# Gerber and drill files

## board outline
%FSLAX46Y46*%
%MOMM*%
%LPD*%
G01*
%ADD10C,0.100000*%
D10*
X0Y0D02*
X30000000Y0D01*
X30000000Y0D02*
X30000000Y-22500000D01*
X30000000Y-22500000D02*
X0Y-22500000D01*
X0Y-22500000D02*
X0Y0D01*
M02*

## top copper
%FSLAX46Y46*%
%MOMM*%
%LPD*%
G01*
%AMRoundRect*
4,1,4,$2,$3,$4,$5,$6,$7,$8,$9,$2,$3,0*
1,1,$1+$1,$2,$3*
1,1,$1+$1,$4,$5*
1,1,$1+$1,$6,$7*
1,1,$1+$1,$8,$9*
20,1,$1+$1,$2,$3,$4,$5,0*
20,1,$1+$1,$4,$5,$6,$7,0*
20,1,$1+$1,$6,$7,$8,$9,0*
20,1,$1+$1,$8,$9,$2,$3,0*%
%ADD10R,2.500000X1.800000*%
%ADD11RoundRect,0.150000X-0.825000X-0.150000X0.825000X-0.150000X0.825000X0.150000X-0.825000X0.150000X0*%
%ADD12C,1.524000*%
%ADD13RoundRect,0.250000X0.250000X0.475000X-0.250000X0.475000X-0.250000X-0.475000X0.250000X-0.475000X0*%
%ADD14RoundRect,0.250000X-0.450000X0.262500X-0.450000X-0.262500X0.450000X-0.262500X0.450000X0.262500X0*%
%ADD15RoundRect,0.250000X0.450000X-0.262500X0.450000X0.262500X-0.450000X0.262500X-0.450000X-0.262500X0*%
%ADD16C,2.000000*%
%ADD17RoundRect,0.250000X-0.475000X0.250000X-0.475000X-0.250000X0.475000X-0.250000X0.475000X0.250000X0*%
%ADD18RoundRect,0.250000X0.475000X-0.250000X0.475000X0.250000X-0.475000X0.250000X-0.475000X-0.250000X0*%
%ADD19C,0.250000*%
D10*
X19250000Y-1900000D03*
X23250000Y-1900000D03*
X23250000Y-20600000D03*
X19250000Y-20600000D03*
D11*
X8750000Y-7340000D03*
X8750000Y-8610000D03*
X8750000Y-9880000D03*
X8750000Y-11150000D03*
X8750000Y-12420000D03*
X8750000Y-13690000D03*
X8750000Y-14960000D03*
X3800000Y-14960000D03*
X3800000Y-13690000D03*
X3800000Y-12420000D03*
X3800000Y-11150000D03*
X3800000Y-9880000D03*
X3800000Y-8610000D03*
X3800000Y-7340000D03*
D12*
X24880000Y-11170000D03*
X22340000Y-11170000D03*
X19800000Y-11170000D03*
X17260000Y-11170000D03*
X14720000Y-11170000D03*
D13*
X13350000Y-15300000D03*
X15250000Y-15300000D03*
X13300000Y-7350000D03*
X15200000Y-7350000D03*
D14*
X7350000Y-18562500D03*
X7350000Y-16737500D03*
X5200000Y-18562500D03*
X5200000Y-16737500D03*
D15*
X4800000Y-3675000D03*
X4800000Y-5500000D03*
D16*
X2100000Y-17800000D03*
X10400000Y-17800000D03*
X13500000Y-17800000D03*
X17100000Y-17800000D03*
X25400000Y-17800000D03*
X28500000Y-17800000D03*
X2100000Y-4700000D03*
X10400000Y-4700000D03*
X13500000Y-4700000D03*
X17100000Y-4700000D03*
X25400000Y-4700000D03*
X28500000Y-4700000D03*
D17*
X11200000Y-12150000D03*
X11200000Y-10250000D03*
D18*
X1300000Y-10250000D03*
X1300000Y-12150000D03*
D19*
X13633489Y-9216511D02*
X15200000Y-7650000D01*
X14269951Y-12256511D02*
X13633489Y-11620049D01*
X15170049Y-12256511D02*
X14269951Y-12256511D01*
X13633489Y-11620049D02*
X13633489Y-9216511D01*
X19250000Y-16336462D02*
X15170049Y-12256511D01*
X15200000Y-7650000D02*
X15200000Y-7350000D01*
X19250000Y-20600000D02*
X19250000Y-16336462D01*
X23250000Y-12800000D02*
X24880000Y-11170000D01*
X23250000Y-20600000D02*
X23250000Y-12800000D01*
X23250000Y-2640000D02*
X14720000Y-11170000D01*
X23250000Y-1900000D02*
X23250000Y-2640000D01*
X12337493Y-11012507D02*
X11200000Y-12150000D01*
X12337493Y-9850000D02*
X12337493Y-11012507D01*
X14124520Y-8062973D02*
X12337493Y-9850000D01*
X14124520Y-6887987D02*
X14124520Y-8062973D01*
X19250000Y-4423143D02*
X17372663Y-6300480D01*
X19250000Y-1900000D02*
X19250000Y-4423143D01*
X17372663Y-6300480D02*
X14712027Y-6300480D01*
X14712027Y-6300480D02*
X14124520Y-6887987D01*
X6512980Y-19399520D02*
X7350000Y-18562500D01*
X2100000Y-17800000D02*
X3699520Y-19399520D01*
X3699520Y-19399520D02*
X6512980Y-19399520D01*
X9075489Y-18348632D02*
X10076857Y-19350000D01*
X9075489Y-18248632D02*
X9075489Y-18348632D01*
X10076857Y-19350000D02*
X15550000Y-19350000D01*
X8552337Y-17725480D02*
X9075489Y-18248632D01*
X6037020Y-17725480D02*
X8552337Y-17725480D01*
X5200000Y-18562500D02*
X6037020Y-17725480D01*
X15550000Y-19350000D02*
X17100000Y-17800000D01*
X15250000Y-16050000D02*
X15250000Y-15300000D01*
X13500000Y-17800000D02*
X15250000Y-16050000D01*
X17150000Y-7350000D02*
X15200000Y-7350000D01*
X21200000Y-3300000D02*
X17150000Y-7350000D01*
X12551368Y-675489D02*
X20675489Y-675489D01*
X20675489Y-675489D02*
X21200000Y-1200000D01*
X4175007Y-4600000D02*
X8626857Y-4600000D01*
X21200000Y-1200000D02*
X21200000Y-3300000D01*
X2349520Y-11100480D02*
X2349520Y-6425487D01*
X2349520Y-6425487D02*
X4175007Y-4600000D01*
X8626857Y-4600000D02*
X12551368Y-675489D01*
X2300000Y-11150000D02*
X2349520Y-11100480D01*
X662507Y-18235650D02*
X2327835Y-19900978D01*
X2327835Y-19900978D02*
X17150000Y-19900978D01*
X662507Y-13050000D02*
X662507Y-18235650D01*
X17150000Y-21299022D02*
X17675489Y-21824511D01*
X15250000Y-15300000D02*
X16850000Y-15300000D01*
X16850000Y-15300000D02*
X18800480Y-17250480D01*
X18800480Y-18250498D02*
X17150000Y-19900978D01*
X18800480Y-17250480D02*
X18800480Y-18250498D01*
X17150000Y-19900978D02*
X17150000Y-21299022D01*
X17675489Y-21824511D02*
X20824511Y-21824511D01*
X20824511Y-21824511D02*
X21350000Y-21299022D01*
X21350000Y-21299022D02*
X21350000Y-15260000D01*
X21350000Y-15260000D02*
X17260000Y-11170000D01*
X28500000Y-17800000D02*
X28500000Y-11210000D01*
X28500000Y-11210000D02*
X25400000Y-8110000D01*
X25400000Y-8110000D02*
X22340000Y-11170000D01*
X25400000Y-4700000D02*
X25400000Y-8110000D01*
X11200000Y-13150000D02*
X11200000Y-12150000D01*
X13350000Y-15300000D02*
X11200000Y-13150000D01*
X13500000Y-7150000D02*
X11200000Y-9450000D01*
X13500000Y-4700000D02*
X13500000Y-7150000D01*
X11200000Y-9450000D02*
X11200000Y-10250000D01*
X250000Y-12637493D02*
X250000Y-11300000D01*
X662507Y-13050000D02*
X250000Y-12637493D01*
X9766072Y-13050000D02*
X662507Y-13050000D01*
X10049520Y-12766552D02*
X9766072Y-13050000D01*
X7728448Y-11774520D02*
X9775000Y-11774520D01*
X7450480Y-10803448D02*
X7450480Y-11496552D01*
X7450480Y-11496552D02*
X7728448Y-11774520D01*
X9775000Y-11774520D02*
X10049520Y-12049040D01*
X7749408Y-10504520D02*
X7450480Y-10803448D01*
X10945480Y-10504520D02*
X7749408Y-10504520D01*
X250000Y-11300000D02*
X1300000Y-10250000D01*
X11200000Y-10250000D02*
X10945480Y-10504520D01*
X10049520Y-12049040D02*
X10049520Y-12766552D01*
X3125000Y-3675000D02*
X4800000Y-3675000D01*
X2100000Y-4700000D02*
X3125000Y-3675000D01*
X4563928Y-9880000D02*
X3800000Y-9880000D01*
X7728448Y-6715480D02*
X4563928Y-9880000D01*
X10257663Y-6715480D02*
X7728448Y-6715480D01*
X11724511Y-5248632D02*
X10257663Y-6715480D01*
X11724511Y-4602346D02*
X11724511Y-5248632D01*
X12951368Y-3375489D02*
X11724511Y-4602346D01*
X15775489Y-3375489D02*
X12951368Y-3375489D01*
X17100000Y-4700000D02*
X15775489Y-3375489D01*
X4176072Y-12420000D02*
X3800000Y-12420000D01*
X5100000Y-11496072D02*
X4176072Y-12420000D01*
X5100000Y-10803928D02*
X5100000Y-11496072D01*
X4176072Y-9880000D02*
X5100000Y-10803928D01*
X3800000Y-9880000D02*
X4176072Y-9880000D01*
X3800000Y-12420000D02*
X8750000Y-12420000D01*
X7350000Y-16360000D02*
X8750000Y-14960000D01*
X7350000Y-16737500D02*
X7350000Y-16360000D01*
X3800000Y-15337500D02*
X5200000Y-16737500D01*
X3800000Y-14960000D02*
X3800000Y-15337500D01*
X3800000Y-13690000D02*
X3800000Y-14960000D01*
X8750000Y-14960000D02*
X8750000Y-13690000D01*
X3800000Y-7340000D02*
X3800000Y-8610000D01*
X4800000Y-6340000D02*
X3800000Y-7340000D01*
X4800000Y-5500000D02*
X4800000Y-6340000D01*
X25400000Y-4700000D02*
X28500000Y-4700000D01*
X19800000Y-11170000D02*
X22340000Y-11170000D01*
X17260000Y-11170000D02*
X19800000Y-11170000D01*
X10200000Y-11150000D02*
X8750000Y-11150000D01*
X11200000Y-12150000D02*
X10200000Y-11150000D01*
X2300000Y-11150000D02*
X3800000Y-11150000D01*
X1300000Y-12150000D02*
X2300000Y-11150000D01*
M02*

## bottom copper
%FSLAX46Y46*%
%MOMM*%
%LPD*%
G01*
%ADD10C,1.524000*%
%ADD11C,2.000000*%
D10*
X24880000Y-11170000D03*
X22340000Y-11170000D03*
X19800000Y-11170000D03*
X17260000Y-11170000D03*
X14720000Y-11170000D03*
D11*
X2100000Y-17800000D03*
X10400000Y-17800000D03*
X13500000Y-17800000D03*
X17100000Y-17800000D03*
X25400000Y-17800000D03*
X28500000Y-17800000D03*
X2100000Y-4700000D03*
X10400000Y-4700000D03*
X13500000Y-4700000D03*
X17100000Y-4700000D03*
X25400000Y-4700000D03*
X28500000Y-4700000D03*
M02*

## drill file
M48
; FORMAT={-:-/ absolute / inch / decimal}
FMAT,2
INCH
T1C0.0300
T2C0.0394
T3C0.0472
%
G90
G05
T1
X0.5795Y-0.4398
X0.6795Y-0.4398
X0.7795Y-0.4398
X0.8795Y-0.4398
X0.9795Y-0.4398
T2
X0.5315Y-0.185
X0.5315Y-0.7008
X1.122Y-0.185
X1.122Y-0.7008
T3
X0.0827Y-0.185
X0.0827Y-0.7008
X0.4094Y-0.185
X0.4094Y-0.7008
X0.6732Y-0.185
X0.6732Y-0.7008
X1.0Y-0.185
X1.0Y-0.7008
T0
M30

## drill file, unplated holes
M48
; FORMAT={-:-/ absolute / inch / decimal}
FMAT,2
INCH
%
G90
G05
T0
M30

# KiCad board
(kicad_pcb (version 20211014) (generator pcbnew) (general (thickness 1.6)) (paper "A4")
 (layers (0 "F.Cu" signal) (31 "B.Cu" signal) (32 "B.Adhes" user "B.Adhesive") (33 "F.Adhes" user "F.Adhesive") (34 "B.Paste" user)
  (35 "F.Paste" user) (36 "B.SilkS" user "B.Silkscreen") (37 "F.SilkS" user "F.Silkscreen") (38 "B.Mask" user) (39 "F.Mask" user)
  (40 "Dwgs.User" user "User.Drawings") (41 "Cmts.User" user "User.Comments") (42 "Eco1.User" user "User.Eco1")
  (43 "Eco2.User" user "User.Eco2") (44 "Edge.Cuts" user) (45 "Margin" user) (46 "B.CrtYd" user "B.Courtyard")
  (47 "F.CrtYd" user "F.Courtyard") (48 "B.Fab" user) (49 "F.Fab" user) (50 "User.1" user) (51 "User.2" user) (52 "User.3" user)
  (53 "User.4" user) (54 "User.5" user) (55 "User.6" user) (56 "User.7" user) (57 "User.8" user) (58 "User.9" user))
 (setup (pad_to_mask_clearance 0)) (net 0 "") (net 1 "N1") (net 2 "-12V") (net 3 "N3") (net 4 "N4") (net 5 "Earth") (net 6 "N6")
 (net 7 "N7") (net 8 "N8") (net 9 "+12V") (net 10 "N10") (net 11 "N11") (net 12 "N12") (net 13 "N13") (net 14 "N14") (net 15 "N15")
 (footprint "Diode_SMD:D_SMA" (layer "F.Cu") (at 21.25 1.9 180)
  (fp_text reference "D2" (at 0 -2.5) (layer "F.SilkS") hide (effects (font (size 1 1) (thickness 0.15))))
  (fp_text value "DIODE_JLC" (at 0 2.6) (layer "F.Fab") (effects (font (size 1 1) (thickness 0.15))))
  (pad "1" smd rect (at -2 0 180) (size 2.5 1.8) (layers "F.Cu" "F.Paste" "F.Mask") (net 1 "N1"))
  (pad "2" smd rect (at 2 0 180) (size 2.5 1.8) (layers "F.Cu" "F.Paste" "F.Mask") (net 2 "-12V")))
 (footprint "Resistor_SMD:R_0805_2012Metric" (layer "F.Cu") (at 7.35 17.65 -90)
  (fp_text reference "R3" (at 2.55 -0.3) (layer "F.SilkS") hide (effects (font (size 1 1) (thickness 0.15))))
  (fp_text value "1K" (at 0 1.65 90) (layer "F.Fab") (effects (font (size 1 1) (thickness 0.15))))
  (pad "1" smd roundrect (at -0.9125 0 270) (size 1.025 1.4) (layers "F.Cu" "F.Paste" "F.Mask") (roundrect_rratio 0.243902439) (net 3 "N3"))
  (pad "2" smd roundrect (at 0.9125 0 270) (size 1.025 1.4) (layers "F.Cu" "F.Paste" "F.Mask") (roundrect_rratio 0.243902439) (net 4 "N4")))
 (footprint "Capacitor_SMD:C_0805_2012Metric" (layer "F.Cu") (at 14.3 15.3 180)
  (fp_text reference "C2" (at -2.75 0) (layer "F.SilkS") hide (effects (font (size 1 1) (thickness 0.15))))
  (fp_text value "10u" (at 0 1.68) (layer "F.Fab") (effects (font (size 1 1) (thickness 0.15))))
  (pad "1" smd roundrect (at -0.95 0 180) (size 1 1.45) (layers "F.Cu" "F.Paste" "F.Mask") (roundrect_rratio 0.25) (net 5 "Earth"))
  (pad "2" smd roundrect (at 0.95 0 180) (size 1 1.45) (layers "F.Cu" "F.Paste" "F.Mask") (roundrect_rratio 0.25) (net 2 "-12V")))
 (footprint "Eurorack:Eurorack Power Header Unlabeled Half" (layer "F.Cu") (at 19.8 9.9 180)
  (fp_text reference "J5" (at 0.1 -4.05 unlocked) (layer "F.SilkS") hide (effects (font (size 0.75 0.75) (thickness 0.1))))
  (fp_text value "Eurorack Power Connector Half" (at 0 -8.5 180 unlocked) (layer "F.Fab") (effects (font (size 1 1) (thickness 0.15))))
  (pad "1" thru_hole circle (at 5.08 -1.27 180) (size 1.524 1.524) (drill 0.762) (layers *.Cu *.Mask) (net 1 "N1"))
  (pad "2" thru_hole circle (at 2.54 -1.27 180) (size 1.524 1.524) (drill 0.762) (layers *.Cu *.Mask) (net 5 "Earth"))
  (pad "3" thru_hole circle (at 0 -1.27 180) (size 1.524 1.524) (drill 0.762) (layers *.Cu *.Mask) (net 5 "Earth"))
  (pad "4" thru_hole circle (at -2.54 -1.27 180) (size 1.524 1.524) (drill 0.762) (layers *.Cu *.Mask) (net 5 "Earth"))
  (pad "5" thru_hole circle (at -5.08 -1.27 180) (size 1.524 1.524) (drill 0.762) (layers *.Cu *.Mask) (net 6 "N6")))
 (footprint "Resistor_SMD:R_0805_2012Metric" (layer "F.Cu") (at 5.2 17.65 -90)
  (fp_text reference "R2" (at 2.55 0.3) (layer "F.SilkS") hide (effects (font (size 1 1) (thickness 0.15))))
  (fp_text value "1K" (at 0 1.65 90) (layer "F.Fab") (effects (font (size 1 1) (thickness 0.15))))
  (pad "1" smd roundrect (at -0.9125 0 270) (size 1.025 1.4) (layers "F.Cu" "F.Paste" "F.Mask") (roundrect_rratio 0.243902439) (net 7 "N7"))
  (pad "2" smd roundrect (at 0.9125 0 270) (size 1.025 1.4) (layers "F.Cu" "F.Paste" "F.Mask") (roundrect_rratio 0.243902439) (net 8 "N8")))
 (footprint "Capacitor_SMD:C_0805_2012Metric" (layer "F.Cu") (at 14.25 7.35 180)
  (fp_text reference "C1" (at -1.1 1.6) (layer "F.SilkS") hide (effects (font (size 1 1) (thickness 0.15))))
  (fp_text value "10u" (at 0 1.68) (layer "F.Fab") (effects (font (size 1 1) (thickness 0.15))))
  (pad "1" smd roundrect (at -0.95 0 180) (size 1 1.45) (layers "F.Cu" "F.Paste" "F.Mask") (roundrect_rratio 0.25) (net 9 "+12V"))
  (pad "2" smd roundrect (at 0.95 0 180) (size 1 1.45) (layers "F.Cu" "F.Paste" "F.Mask") (roundrect_rratio 0.25) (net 5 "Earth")))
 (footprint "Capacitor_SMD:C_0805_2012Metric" (layer "F.Cu") (at 11.2 11.2 -90)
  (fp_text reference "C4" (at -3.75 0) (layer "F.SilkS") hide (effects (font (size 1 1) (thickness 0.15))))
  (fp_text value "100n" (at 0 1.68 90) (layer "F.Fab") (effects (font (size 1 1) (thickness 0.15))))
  (pad "1" smd roundrect (at -0.95 0 270) (size 1 1.45) (layers "F.Cu" "F.Paste" "F.Mask") (roundrect_rratio 0.25) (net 5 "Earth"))
  (pad "2" smd roundrect (at 0.95 0 270) (size 1 1.45) (layers "F.Cu" "F.Paste" "F.Mask") (roundrect_rratio 0.25) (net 2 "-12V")))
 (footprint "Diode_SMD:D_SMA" (layer "F.Cu") (at 21.25 20.6)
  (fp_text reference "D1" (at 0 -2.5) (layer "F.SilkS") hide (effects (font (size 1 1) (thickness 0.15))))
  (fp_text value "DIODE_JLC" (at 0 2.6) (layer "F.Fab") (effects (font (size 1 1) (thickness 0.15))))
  (pad "1" smd rect (at -2 0) (size 2.5 1.8) (layers "F.Cu" "F.Paste" "F.Mask") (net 9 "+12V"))
  (pad "2" smd rect (at 2 0) (size 2.5 1.8) (layers "F.Cu" "F.Paste" "F.Mask") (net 6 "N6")))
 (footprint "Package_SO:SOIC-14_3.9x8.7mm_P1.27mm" (layer "F.Cu") (at 6.275 11.15)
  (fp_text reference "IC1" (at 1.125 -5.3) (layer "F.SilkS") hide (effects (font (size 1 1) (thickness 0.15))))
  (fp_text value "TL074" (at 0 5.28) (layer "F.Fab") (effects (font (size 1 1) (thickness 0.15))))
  (pad "1" smd roundrect (at -2.475 -3.81) (size 1.95 0.6) (layers "F.Cu" "F.Paste" "F.Mask") (roundrect_rratio 0.25) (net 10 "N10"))
  (pad "2" smd roundrect (at -2.475 -2.54) (size 1.95 0.6) (layers "F.Cu" "F.Paste" "F.Mask") (roundrect_rratio 0.25) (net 10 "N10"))
  (pad "3" smd roundrect (at -2.475 -1.27) (size 1.95 0.6) (layers "F.Cu" "F.Paste" "F.Mask") (roundrect_rratio 0.25) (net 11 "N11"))
  (pad "4" smd roundrect (at -2.475 0) (size 1.95 0.6) (layers "F.Cu" "F.Paste" "F.Mask") (roundrect_rratio 0.25) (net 9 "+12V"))
  (pad "5" smd roundrect (at -2.475 1.27) (size 1.95 0.6) (layers "F.Cu" "F.Paste" "F.Mask") (roundrect_rratio 0.25) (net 11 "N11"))
  (pad "6" smd roundrect (at -2.475 2.54) (size 1.95 0.6) (layers "F.Cu" "F.Paste" "F.Mask") (roundrect_rratio 0.25) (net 7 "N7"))
  (pad "7" smd roundrect (at -2.475 3.81) (size 1.95 0.6) (layers "F.Cu" "F.Paste" "F.Mask") (roundrect_rratio 0.25) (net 7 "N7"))
  (pad "8" smd roundrect (at 2.475 3.81) (size 1.95 0.6) (layers "F.Cu" "F.Paste" "F.Mask") (roundrect_rratio 0.25) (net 3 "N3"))
  (pad "9" smd roundrect (at 2.475 2.54) (size 1.95 0.6) (layers "F.Cu" "F.Paste" "F.Mask") (roundrect_rratio 0.25) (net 3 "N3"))
  (pad "10" smd roundrect (at 2.475 1.27) (size 1.95 0.6) (layers "F.Cu" "F.Paste" "F.Mask") (roundrect_rratio 0.25) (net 11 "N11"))
  (pad "11" smd roundrect (at 2.475 0) (size 1.95 0.6) (layers "F.Cu" "F.Paste" "F.Mask") (roundrect_rratio 0.25) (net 2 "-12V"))
  (pad "12" smd roundrect (at 2.475 -1.27) (size 1.95 0.6) (layers "F.Cu" "F.Paste" "F.Mask") (roundrect_rratio 0.25))
  (pad "13" smd roundrect (at 2.475 -2.54) (size 1.95 0.6) (layers "F.Cu" "F.Paste" "F.Mask") (roundrect_rratio 0.25))
  (pad "14" smd roundrect (at 2.475 -3.81) (size 1.95 0.6) (layers "F.Cu" "F.Paste" "F.Mask") (roundrect_rratio 0.25)))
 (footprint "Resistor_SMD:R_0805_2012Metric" (layer "F.Cu") (at 4.8 4.5875 90)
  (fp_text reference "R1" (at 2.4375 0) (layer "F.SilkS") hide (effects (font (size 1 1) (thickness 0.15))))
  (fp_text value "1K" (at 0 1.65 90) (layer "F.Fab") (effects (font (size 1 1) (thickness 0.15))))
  (pad "1" smd roundrect (at -0.9125 0 90) (size 1.025 1.4) (layers "F.Cu" "F.Paste" "F.Mask") (roundrect_rratio 0.243902439) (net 10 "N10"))
  (pad "2" smd roundrect (at 0.9125 0 90) (size 1.025 1.4) (layers "F.Cu" "F.Paste" "F.Mask") (roundrect_rratio 0.243902439) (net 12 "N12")))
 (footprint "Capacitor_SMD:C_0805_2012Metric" (layer "F.Cu") (at 1.3 11.2 90)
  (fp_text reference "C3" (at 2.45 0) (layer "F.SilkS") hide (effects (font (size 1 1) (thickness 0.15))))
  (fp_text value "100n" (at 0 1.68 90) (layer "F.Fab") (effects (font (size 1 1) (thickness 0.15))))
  (pad "1" smd roundrect (at -0.95 0 90) (size 1 1.45) (layers "F.Cu" "F.Paste" "F.Mask") (roundrect_rratio 0.25) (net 9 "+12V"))
  (pad "2" smd roundrect (at 0.95 0 90) (size 1 1.45) (layers "F.Cu" "F.Paste" "F.Mask") (roundrect_rratio 0.25) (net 5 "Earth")))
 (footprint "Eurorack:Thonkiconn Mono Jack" (layer "B.Cu") (at 22.5 4.7 180)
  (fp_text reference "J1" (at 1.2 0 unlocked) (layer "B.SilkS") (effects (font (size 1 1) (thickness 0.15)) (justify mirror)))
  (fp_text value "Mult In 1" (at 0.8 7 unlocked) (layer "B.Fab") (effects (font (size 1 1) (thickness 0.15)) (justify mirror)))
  (pad "1" thru_hole circle (at -6 0 180) (size 2 2) (drill 1) (layers *.Cu *.Mask) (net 5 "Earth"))
  (pad "2" thru_hole circle (at -2.9 0 180) (size 2 2) (drill 1.2) (layers *.Cu *.Mask) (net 5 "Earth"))
  (pad "3" thru_hole circle (at 5.4 0 180) (size 2 2) (drill 1.2) (layers *.Cu *.Mask) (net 11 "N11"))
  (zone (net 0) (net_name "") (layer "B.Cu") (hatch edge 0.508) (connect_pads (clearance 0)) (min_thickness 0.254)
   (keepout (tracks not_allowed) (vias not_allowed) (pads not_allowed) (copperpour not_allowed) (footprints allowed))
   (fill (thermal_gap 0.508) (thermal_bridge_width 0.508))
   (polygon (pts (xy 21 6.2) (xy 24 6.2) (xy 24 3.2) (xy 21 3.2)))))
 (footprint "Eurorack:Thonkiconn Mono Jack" (layer "B.Cu") (at 7.5 17.8 180)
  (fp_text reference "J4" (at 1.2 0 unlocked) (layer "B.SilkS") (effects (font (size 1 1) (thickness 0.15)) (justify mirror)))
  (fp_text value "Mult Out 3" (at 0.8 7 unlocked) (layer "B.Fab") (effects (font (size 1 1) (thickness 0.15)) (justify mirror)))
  (pad "1" thru_hole circle (at -6 0 180) (size 2 2) (drill 1) (layers *.Cu *.Mask) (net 5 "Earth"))
  (pad "2" thru_hole circle (at -2.9 0 180) (size 2 2) (drill 1.2) (layers *.Cu *.Mask) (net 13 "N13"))
  (pad "3" thru_hole circle (at 5.4 0 180) (size 2 2) (drill 1.2) (layers *.Cu *.Mask) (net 4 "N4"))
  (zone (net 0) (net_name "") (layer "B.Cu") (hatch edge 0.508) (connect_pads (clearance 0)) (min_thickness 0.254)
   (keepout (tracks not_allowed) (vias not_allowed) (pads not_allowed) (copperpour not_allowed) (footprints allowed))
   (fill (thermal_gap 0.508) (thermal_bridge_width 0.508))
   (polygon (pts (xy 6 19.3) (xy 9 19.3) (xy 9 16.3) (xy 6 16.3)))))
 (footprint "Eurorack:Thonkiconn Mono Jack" (layer "B.Cu") (at 22.5 17.8 180)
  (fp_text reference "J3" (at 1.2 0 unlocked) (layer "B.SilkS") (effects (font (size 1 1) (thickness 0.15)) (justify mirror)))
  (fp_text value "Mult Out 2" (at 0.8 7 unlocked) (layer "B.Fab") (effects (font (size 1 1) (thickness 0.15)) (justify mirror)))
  (pad "1" thru_hole circle (at -6 0 180) (size 2 2) (drill 1) (layers *.Cu *.Mask) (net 5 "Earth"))
  (pad "2" thru_hole circle (at -2.9 0 180) (size 2 2) (drill 1.2) (layers *.Cu *.Mask) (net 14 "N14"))
  (pad "3" thru_hole circle (at 5.4 0 180) (size 2 2) (drill 1.2) (layers *.Cu *.Mask) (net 8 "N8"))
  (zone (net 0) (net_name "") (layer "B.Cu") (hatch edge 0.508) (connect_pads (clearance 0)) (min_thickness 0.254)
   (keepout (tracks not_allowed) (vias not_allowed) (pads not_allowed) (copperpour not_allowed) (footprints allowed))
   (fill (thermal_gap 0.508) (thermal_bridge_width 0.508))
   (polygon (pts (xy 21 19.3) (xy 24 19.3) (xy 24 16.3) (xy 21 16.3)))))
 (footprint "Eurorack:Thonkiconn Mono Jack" (layer "B.Cu") (at 7.5 4.7 180)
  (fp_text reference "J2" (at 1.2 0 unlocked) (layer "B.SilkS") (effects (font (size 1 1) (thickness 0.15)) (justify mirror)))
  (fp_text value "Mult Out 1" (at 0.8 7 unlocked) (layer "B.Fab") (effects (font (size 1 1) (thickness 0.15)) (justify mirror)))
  (pad "1" thru_hole circle (at -6 0 180) (size 2 2) (drill 1) (layers *.Cu *.Mask) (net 5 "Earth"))
  (pad "2" thru_hole circle (at -2.9 0 180) (size 2 2) (drill 1.2) (layers *.Cu *.Mask) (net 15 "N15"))
  (pad "3" thru_hole circle (at 5.4 0 180) (size 2 2) (drill 1.2) (layers *.Cu *.Mask) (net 12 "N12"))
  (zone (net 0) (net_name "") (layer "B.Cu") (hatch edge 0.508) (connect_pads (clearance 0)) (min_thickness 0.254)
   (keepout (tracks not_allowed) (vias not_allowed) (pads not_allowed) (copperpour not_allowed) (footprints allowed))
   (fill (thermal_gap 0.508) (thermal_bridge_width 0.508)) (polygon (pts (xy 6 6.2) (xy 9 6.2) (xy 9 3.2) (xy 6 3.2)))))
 (gr_rect (start 0 0) (end 30 22.5) (layer "Edge.Cuts") (width 0.1) (fill none))
 (segment (start 2.34952 6.425487) (end 4.175007 4.6) (width 0.25) (layer "F.Cu") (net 9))
 (segment (start 2.3 11.15) (end 2.34952 11.10048) (width 0.25) (layer "F.Cu") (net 9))
 (segment (start 20.675489 0.675489) (end 21.2 1.2) (width 0.25) (layer "F.Cu") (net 9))
 (segment (start 8.626857 4.6) (end 12.551368 0.675489) (width 0.25) (layer "F.Cu") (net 9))
 (segment (start 15.170049 12.256511) (end 14.269951 12.256511) (width 0.25) (layer "F.Cu") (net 9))
 (segment (start 21.2 3.3) (end 17.15 7.35) (width 0.25) (layer "F.Cu") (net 9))
 (segment (start 21.2 1.2) (end 21.2 3.3) (width 0.25) (layer "F.Cu") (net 9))
 (segment (start 12.551368 0.675489) (end 20.675489 0.675489) (width 0.25) (layer "F.Cu") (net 9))
 (segment (start 19.25 20.6) (end 19.25 16.336462) (width 0.25) (layer "F.Cu") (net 9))
 (segment (start 14.269951 12.256511) (end 13.633489 11.620049) (width 0.25) (layer "F.Cu") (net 9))
 (segment (start 15.2 7.65) (end 15.2 7.35) (width 0.25) (layer "F.Cu") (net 9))
 (segment (start 13.633489 9.216511) (end 15.2 7.65) (width 0.25) (layer "F.Cu") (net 9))
 (segment (start 19.25 16.336462) (end 15.170049 12.256511) (width 0.25) (layer "F.Cu") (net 9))
 (segment (start 1.3 12.15) (end 2.3 11.15) (width 0.25) (layer "F.Cu") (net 9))
 (segment (start 17.15 7.35) (end 15.2 7.35) (width 0.25) (layer "F.Cu") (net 9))
 (segment (start 2.3 11.15) (end 3.8 11.15) (width 0.25) (layer "F.Cu") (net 9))
 (segment (start 13.633489 11.620049) (end 13.633489 9.216511) (width 0.25) (layer "F.Cu") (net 9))
 (segment (start 4.175007 4.6) (end 8.626857 4.6) (width 0.25) (layer "F.Cu") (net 9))
 (segment (start 2.34952 11.10048) (end 2.34952 6.425487) (width 0.25) (layer "F.Cu") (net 9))
 (segment (start 9.775 11.77452) (end 10.04952 12.04904) (width 0.25) (layer "F.Cu") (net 5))
 (segment (start 10.04952 12.04904) (end 10.04952 12.766552) (width 0.25) (layer "F.Cu") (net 5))
 (segment (start 25.4 4.7) (end 28.5 4.7) (width 0.25) (layer "F.Cu") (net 5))
 (segment (start 0.25 11.3) (end 1.3 10.25) (width 0.25) (layer "F.Cu") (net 5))
 (segment (start 21.35 21.299022) (end 21.35 15.26) (width 0.25) (layer "F.Cu") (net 5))
 (segment (start 7.45048 11.496552) (end 7.728448 11.77452) (width 0.25) (layer "F.Cu") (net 5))
 (segment (start 2.327835 19.900978) (end 17.15 19.900978) (width 0.25) (layer "F.Cu") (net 5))
 (segment (start 18.80048 17.25048) (end 18.80048 18.250498) (width 0.25) (layer "F.Cu") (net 5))
 (segment (start 11.2 10.25) (end 10.94548 10.50452) (width 0.25) (layer "F.Cu") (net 5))
 (segment (start 7.45048 10.803448) (end 7.45048 11.496552) (width 0.25) (layer "F.Cu") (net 5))
 (segment (start 20.824511 21.824511) (end 21.35 21.299022) (width 0.25) (layer "F.Cu") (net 5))
 (segment (start 25.4 4.7) (end 25.4 8.11) (width 0.25) (layer "F.Cu") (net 5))
 (segment (start 19.8 11.17) (end 22.34 11.17) (width 0.25) (layer "F.Cu") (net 5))
 (segment (start 17.675489 21.824511) (end 20.824511 21.824511) (width 0.25) (layer "F.Cu") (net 5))
 (segment (start 25.4 8.11) (end 22.34 11.17) (width 0.25) (layer "F.Cu") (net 5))
 (segment (start 28.5 11.21) (end 25.4 8.11) (width 0.25) (layer "F.Cu") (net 5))
 (segment (start 21.35 15.26) (end 17.26 11.17) (width 0.25) (layer "F.Cu") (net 5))
 (segment (start 0.662507 13.05) (end 0.662507 18.23565) (width 0.25) (layer "F.Cu") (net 5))
 (segment (start 13.5 4.7) (end 13.5 7.15) (width 0.25) (layer "F.Cu") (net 5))
 (segment (start 28.5 17.8) (end 28.5 11.21) (width 0.25) (layer "F.Cu") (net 5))
 (segment (start 13.5 17.8) (end 15.25 16.05) (width 0.25) (layer "F.Cu") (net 5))
 (segment (start 17.15 19.900978) (end 17.15 21.299022) (width 0.25) (layer "F.Cu") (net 5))
 (segment (start 13.5 7.15) (end 11.2 9.45) (width 0.25) (layer "F.Cu") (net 5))
 (segment (start 11.2 9.45) (end 11.2 10.25) (width 0.25) (layer "F.Cu") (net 5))
 (segment (start 10.94548 10.50452) (end 7.749408 10.50452) (width 0.25) (layer "F.Cu") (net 5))
 (segment (start 17.26 11.17) (end 19.8 11.17) (width 0.25) (layer "F.Cu") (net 5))
 (segment (start 0.25 12.637493) (end 0.25 11.3) (width 0.25) (layer "F.Cu") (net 5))
 (segment (start 10.04952 12.766552) (end 9.766072 13.05) (width 0.25) (layer "F.Cu") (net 5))
 (segment (start 7.728448 11.77452) (end 9.775 11.77452) (width 0.25) (layer "F.Cu") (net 5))
 (segment (start 18.80048 18.250498) (end 17.15 19.900978) (width 0.25) (layer "F.Cu") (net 5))
 (segment (start 16.85 15.3) (end 18.80048 17.25048) (width 0.25) (layer "F.Cu") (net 5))
 (segment (start 0.662507 13.05) (end 0.25 12.637493) (width 0.25) (layer "F.Cu") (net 5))
 (segment (start 17.15 21.299022) (end 17.675489 21.824511) (width 0.25) (layer "F.Cu") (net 5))
 (segment (start 0.662507 18.23565) (end 2.327835 19.900978) (width 0.25) (layer "F.Cu") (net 5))
 (segment (start 15.25 15.3) (end 16.85 15.3) (width 0.25) (layer "F.Cu") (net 5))
 (segment (start 9.766072 13.05) (end 0.662507 13.05) (width 0.25) (layer "F.Cu") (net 5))
 (segment (start 15.25 16.05) (end 15.25 15.3) (width 0.25) (layer "F.Cu") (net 5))
 (segment (start 7.749408 10.50452) (end 7.45048 10.803448) (width 0.25) (layer "F.Cu") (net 5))
 (segment (start 10.2 11.15) (end 8.75 11.15) (width 0.25) (layer "F.Cu") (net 2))
 (segment (start 13.35 15.3) (end 11.2 13.15) (width 0.25) (layer "F.Cu") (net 2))
 (segment (start 19.25 4.423143) (end 17.372663 6.30048) (width 0.25) (layer "F.Cu") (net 2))
 (segment (start 17.372663 6.30048) (end 14.712027 6.30048) (width 0.25) (layer "F.Cu") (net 2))
 (segment (start 12.337493 11.012507) (end 11.2 12.15) (width 0.25) (layer "F.Cu") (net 2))
 (segment (start 11.2 13.15) (end 11.2 12.15) (width 0.25) (layer "F.Cu") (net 2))
 (segment (start 14.712027 6.30048) (end 14.12452 6.887987) (width 0.25) (layer "F.Cu") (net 2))
 (segment (start 14.12452 8.062973) (end 12.337493 9.85) (width 0.25) (layer "F.Cu") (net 2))
 (segment (start 19.25 1.9) (end 19.25 4.423143) (width 0.25) (layer "F.Cu") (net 2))
 (segment (start 14.12452 6.887987) (end 14.12452 8.062973) (width 0.25) (layer "F.Cu") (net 2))
 (segment (start 12.337493 9.85) (end 12.337493 11.012507) (width 0.25) (layer "F.Cu") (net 2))
 (segment (start 11.2 12.15) (end 10.2 11.15) (width 0.25) (layer "F.Cu") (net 2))
 (segment (start 2.1 4.7) (end 3.125 3.675) (width 0.25) (layer "F.Cu") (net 12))
 (segment (start 3.125 3.675) (end 4.8 3.675) (width 0.25) (layer "F.Cu") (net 12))
 (segment (start 15.55 19.35) (end 17.1 17.8) (width 0.25) (layer "F.Cu") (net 8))
 (segment (start 8.552337 17.72548) (end 9.075489 18.248632) (width 0.25) (layer "F.Cu") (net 8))
 (segment (start 5.2 18.5625) (end 6.03702 17.72548) (width 0.25) (layer "F.Cu") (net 8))
 (segment (start 10.076857 19.35) (end 15.55 19.35) (width 0.25) (layer "F.Cu") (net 8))
 (segment (start 6.03702 17.72548) (end 8.552337 17.72548) (width 0.25) (layer "F.Cu") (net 8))
 (segment (start 9.075489 18.348632) (end 10.076857 19.35) (width 0.25) (layer "F.Cu") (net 8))
 (segment (start 9.075489 18.248632) (end 9.075489 18.348632) (width 0.25) (layer "F.Cu") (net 8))
 (segment (start 3.69952 19.39952) (end 6.51298 19.39952) (width 0.25) (layer "F.Cu") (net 4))
 (segment (start 6.51298 19.39952) (end 7.35 18.5625) (width 0.25) (layer "F.Cu") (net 4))
 (segment (start 2.1 17.8) (end 3.69952 19.39952) (width 0.25) (layer "F.Cu") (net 4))
 (segment (start 8.75 14.96) (end 8.75 13.69) (width 0.25) (layer "F.Cu") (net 3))
 (segment (start 7.35 16.36) (end 8.75 14.96) (width 0.25) (layer "F.Cu") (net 3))
 (segment (start 7.35 16.7375) (end 7.35 16.36) (width 0.25) (layer "F.Cu") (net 3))
 (segment (start 3.8 14.96) (end 3.8 15.3375) (width 0.25) (layer "F.Cu") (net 7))
 (segment (start 3.8 15.3375) (end 5.2 16.7375) (width 0.25) (layer "F.Cu") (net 7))
 (segment (start 3.8 13.69) (end 3.8 14.96) (width 0.25) (layer "F.Cu") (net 7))
 (segment (start 4.8 6.34) (end 3.8 7.34) (width 0.25) (layer "F.Cu") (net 10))
 (segment (start 3.8 7.34) (end 3.8 8.61) (width 0.25) (layer "F.Cu") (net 10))
 (segment (start 4.8 5.5) (end 4.8 6.34) (width 0.25) (layer "F.Cu") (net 10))
 (segment (start 23.25 12.8) (end 24.88 11.17) (width 0.25) (layer "F.Cu") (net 6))
 (segment (start 23.25 20.6) (end 23.25 12.8) (width 0.25) (layer "F.Cu") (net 6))
 (segment (start 23.25 1.9) (end 23.25 2.64) (width 0.25) (layer "F.Cu") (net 1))
 (segment (start 23.25 2.64) (end 14.72 11.17) (width 0.25) (layer "F.Cu") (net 1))
 (segment (start 3.8 9.88) (end 4.176072 9.88) (width 0.25) (layer "F.Cu") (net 11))
 (segment (start 12.951368 3.375489) (end 11.724511 4.602346) (width 0.25) (layer "F.Cu") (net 11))
 (segment (start 3.8 12.42) (end 8.75 12.42) (width 0.25) (layer "F.Cu") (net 11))
 (segment (start 4.176072 12.42) (end 3.8 12.42) (width 0.25) (layer "F.Cu") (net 11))
 (segment (start 11.724511 4.602346) (end 11.724511 5.248632) (width 0.25) (layer "F.Cu") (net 11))
 (segment (start 15.775489 3.375489) (end 12.951368 3.375489) (width 0.25) (layer "F.Cu") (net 11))
 (segment (start 4.176072 9.88) (end 5.1 10.803928) (width 0.25) (layer "F.Cu") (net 11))
 (segment (start 5.1 11.496072) (end 4.176072 12.42) (width 0.25) (layer "F.Cu") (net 11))
 (segment (start 4.563928 9.88) (end 3.8 9.88) (width 0.25) (layer "F.Cu") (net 11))
 (segment (start 11.724511 5.248632) (end 10.257663 6.71548) (width 0.25) (layer "F.Cu") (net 11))
 (segment (start 7.728448 6.71548) (end 4.563928 9.88) (width 0.25) (layer "F.Cu") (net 11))
 (segment (start 17.1 4.7) (end 15.775489 3.375489) (width 0.25) (layer "F.Cu") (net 11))
 (segment (start 5.1 10.803928) (end 5.1 11.496072) (width 0.25) (layer "F.Cu") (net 11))
 (segment (start 10.257663 6.71548) (end 7.728448 6.71548) (width 0.25) (layer "F.Cu") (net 11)))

